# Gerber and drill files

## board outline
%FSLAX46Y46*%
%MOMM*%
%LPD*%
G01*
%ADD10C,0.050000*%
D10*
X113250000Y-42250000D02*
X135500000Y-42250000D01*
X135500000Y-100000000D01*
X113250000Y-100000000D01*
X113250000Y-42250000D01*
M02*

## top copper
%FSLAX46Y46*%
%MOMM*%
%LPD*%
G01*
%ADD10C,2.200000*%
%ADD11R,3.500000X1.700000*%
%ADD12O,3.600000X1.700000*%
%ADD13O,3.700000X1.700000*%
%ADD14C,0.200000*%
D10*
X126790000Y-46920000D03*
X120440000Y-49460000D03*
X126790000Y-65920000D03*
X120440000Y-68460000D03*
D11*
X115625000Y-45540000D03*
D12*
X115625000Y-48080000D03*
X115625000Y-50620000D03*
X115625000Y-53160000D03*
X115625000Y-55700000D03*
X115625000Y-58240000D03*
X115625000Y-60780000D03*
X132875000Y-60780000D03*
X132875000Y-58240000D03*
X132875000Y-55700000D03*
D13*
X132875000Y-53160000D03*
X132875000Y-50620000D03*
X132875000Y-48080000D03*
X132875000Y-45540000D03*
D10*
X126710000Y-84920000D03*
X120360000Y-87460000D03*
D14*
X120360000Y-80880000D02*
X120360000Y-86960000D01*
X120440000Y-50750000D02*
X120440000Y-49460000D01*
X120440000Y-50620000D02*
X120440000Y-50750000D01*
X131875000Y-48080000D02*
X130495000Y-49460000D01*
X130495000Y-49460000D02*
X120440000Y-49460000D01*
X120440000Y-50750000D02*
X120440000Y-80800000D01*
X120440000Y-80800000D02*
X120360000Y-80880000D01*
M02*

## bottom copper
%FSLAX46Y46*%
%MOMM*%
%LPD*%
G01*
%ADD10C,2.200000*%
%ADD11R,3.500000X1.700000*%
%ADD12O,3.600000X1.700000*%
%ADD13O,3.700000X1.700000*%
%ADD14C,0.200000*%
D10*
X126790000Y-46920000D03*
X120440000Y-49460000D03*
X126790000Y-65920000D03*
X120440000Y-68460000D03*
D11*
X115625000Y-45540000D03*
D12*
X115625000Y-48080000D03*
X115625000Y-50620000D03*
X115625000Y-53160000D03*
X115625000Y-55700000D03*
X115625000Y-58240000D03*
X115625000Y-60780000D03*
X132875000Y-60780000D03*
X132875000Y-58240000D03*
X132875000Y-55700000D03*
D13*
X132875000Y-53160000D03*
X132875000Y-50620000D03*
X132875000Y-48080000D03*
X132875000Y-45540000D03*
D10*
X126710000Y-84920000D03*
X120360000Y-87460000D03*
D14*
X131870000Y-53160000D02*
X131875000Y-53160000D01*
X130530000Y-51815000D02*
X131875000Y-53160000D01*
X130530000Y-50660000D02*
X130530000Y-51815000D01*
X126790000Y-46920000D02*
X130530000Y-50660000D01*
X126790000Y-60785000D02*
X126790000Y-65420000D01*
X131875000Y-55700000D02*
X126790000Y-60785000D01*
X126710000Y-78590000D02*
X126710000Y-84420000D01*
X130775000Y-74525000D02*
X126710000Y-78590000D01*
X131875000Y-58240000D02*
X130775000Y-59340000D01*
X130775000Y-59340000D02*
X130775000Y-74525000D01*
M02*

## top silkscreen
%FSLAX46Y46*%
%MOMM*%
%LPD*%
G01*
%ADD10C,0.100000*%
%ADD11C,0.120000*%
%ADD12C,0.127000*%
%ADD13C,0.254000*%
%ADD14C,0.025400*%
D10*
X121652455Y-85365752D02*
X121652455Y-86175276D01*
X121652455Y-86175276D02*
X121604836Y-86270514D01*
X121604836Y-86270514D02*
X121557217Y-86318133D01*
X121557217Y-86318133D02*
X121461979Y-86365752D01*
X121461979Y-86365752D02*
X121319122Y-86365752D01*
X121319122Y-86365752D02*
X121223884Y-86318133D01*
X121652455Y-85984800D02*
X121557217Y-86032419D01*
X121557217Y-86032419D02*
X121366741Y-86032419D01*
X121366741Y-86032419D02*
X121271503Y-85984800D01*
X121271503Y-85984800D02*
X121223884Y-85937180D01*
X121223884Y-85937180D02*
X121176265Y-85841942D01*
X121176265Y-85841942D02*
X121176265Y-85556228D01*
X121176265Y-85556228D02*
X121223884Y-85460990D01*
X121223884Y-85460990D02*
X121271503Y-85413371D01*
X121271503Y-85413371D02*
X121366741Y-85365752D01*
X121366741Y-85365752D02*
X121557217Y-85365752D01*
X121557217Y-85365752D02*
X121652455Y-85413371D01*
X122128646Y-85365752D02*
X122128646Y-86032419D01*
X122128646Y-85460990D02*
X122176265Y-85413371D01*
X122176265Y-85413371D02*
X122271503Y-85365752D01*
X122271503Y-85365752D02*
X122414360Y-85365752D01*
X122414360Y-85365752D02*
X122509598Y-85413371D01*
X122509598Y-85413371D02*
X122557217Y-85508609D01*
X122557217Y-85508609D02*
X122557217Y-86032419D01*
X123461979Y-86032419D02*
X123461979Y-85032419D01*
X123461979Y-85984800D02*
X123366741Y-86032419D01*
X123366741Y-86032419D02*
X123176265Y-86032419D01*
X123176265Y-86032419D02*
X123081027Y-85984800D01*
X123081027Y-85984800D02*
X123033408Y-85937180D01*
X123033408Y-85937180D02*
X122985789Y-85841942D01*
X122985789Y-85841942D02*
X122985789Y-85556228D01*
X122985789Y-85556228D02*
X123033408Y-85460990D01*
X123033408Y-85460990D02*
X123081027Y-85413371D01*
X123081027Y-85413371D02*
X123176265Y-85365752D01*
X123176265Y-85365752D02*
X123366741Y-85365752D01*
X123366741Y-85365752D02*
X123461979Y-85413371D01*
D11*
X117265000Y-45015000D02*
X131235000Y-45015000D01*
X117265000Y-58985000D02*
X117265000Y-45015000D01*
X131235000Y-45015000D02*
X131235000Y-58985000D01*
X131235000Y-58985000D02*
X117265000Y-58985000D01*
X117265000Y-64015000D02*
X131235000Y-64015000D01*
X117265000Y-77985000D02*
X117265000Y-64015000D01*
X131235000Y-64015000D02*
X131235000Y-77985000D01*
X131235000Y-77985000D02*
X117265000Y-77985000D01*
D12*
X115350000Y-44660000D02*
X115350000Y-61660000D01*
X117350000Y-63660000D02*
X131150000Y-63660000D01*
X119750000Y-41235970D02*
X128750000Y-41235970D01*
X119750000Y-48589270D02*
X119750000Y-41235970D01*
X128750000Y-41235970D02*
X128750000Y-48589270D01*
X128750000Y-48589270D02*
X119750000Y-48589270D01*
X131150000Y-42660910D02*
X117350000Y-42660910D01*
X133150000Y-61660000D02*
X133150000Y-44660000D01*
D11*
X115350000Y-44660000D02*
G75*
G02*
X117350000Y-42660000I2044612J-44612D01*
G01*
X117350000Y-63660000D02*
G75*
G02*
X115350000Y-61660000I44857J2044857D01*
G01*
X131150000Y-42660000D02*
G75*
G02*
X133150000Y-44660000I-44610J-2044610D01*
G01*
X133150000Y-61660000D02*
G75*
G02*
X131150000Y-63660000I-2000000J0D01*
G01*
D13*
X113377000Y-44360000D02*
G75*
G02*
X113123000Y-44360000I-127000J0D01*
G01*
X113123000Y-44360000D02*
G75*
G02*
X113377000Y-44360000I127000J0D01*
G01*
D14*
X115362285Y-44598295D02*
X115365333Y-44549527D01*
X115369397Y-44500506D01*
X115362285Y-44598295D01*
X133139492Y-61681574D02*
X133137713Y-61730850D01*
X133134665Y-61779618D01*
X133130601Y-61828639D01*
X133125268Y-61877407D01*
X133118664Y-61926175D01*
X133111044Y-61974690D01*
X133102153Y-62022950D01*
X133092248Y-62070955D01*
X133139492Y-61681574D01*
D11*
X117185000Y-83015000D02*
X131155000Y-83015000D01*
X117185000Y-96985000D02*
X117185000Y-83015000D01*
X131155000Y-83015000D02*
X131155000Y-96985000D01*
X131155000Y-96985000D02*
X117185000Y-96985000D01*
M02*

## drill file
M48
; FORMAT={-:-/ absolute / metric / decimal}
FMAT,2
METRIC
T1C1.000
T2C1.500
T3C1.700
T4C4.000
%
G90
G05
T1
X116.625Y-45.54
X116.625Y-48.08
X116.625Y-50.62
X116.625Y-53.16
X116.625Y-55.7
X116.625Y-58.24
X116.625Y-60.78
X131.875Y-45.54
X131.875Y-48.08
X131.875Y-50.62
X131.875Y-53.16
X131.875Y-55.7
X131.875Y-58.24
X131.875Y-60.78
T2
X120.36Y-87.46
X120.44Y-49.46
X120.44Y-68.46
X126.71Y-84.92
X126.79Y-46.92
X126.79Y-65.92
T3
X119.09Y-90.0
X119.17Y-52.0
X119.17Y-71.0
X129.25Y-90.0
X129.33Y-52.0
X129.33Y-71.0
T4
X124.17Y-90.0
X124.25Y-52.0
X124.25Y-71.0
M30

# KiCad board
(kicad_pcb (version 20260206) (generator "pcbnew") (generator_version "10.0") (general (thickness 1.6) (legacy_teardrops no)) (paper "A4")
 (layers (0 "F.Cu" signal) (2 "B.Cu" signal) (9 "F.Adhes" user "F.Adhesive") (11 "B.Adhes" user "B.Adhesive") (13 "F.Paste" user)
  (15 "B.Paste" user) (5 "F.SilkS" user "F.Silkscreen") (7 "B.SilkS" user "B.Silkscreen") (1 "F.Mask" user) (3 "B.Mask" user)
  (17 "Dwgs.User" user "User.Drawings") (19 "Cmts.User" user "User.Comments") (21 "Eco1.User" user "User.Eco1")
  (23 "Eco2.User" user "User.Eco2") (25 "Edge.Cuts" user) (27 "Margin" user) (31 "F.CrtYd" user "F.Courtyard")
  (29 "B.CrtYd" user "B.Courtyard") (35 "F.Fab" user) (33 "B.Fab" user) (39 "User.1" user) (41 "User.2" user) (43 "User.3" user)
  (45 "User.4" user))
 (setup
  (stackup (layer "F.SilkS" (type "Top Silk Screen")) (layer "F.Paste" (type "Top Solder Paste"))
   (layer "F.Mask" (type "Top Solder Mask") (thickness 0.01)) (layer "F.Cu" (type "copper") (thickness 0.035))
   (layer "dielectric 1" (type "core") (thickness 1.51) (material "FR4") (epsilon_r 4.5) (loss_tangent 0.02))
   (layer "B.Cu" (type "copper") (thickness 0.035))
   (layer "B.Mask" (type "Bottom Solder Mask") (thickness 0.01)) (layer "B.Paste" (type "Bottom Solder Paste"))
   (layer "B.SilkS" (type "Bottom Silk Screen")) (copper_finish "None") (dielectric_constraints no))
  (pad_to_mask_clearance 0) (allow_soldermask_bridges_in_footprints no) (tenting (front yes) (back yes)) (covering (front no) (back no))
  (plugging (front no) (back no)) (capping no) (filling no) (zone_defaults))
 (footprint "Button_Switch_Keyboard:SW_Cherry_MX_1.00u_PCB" (layer "F.Cu") (at 126.79 46.92)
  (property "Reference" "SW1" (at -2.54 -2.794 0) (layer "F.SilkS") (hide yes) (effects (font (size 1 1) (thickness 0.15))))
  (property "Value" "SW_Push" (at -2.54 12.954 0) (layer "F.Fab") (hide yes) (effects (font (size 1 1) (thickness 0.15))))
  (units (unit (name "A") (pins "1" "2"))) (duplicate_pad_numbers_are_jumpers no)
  (fp_line (start -9.525 -1.905) (end 4.445 -1.905) (stroke (width 0.12) (type solid)) (layer "F.SilkS"))
  (fp_line (start -9.525 12.065) (end -9.525 -1.905) (stroke (width 0.12) (type solid)) (layer "F.SilkS"))
  (fp_line (start 4.445 -1.905) (end 4.445 12.065) (stroke (width 0.12) (type solid)) (layer "F.SilkS"))
  (fp_line (start 4.445 12.065) (end -9.525 12.065) (stroke (width 0.12) (type solid)) (layer "F.SilkS"))
  (pad "" np_thru_hole circle (at -7.62 5.08) (size 1.7 1.7) (drill 1.7) (layers "*.Cu" "*.Mask"))
  (pad "" np_thru_hole circle (at -2.54 5.08) (size 4 4) (drill 4) (layers "*.Cu" "*.Mask"))
  (pad "" np_thru_hole circle (at 2.54 5.08) (size 1.7 1.7) (drill 1.7) (layers "*.Cu" "*.Mask"))
  (pad "1" thru_hole circle (at 0 0) (size 2.2 2.2) (drill 1.5) (layers "*.Cu" "*.Mask") (remove_unused_layers no)
   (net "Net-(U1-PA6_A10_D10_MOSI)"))
  (pad "2" thru_hole circle (at -6.35 2.54) (size 2.2 2.2) (drill 1.5) (layers "*.Cu" "*.Mask") (remove_unused_layers no) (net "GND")))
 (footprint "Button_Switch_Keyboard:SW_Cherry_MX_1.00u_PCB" (layer "F.Cu") (at 126.79 65.92)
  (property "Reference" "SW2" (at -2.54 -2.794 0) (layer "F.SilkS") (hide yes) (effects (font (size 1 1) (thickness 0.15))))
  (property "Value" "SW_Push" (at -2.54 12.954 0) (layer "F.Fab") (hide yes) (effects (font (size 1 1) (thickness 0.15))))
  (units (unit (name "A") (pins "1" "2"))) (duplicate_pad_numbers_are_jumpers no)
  (fp_line (start -9.525 -1.905) (end 4.445 -1.905) (stroke (width 0.12) (type solid)) (layer "F.SilkS"))
  (fp_line (start -9.525 12.065) (end -9.525 -1.905) (stroke (width 0.12) (type solid)) (layer "F.SilkS"))
  (fp_line (start 4.445 -1.905) (end 4.445 12.065) (stroke (width 0.12) (type solid)) (layer "F.SilkS"))
  (fp_line (start 4.445 12.065) (end -9.525 12.065) (stroke (width 0.12) (type solid)) (layer "F.SilkS"))
  (pad "" np_thru_hole circle (at -7.62 5.08) (size 1.7 1.7) (drill 1.7) (layers "*.Cu" "*.Mask"))
  (pad "" np_thru_hole circle (at -2.54 5.08) (size 4 4) (drill 4) (layers "*.Cu" "*.Mask"))
  (pad "" np_thru_hole circle (at 2.54 5.08) (size 1.7 1.7) (drill 1.7) (layers "*.Cu" "*.Mask"))
  (pad "1" thru_hole circle (at 0 0) (size 2.2 2.2) (drill 1.5) (layers "*.Cu" "*.Mask") (remove_unused_layers no)
   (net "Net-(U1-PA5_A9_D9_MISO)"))
  (pad "2" thru_hole circle (at -6.35 2.54) (size 2.2 2.2) (drill 1.5) (layers "*.Cu" "*.Mask") (remove_unused_layers no) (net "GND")))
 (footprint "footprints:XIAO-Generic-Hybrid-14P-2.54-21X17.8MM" (layer "F.Cu") (at 124.25 53.16)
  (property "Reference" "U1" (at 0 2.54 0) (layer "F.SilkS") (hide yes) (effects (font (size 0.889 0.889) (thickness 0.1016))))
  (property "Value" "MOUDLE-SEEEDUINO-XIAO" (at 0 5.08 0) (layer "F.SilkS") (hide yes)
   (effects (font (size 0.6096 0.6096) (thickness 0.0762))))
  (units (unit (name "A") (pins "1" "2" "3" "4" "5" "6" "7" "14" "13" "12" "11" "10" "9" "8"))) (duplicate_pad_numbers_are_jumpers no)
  (fp_line (start -8.9 -8.5) (end -8.9 8.5) (stroke (width 0.127) (type solid)) (layer "F.SilkS"))
  (fp_line (start -6.9 10.5) (end 6.9 10.5) (stroke (width 0.127) (type solid)) (layer "F.SilkS"))
  (fp_line (start -4.5 -11.92403) (end 4.5 -11.92403) (stroke (width 0.127) (type solid)) (layer "F.SilkS"))
  (fp_line (start -4.5 -4.57073) (end -4.5 -11.92403) (stroke (width 0.127) (type solid)) (layer "F.SilkS"))
  (fp_line (start 4.5 -11.92403) (end 4.5 -4.57073) (stroke (width 0.127) (type solid)) (layer "F.SilkS"))
  (fp_line (start 4.5 -4.57073) (end -4.5 -4.57073) (stroke (width 0.127) (type solid)) (layer "F.SilkS"))
  (fp_line (start 6.9 -10.49909) (end -6.9 -10.49909) (stroke (width 0.127) (type solid)) (layer "F.SilkS"))
  (fp_line (start 8.9 8.5) (end 8.9 -8.5) (stroke (width 0.127) (type solid)) (layer "F.SilkS"))
  (fp_arc (start -8.9 -8.5) (mid -8.301491 -9.901491) (end -6.9 -10.5) (stroke (width 0.12) (type solid)) (layer "F.SilkS"))
  (fp_arc (start -6.9 10.5) (mid -8.301423 9.901423) (end -8.9 8.5) (stroke (width 0.12) (type solid)) (layer "F.SilkS"))
  (fp_arc (start 6.9 -10.5) (mid 8.301491 -9.901491) (end 8.9 -8.5) (stroke (width 0.12) (type solid)) (layer "F.SilkS"))
  (fp_arc (start 8.9 8.5) (mid 8.314214 9.914214) (end 6.9 10.5) (stroke (width 0.12) (type solid)) (layer "F.SilkS"))
  (fp_circle (center -11 -8.8) (end -11 -9.054) (stroke (width 0) (type solid)) (fill yes) (layer "F.SilkS"))
  (fp_poly
   (pts (xy -8.887715 -8.561705) (xy -8.884667 -8.610473) (xy -8.880603 -8.659494)) (stroke (width 0.0254) (type solid)) (fill no)
   (layer "F.SilkS"))
  (fp_poly
   (pts (xy 8.889492 8.521574) (xy 8.887713 8.57085) (xy 8.884665 8.619618) (xy 8.880601 8.668639) (xy 8.875268 8.717407)
    (xy 8.868664 8.766175) (xy 8.861044 8.81469) (xy 8.852153 8.86295) (xy 8.842248 8.910955))
   (stroke (width 0.0254) (type solid)) (fill no) (layer "F.SilkS"))
  (pad "1" thru_hole rect (at -7.625 -7.62) (size 3.5 1.7) (drill 1 (offset -1 0)) (layers "*.Cu" "*.Mask") (remove_unused_layers no)
   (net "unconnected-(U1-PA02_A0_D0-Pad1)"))
  (pad "2" thru_hole oval (at -7.625 -5.08) (size 3.6 1.7) (drill 1 (offset -1 0)) (layers "*.Cu" "*.Mask") (remove_unused_layers no)
   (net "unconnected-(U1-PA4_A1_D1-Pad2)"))
  (pad "3" thru_hole oval (at -7.625 -2.54) (size 3.6 1.7) (drill 1 (offset -1 0)) (layers "*.Cu" "*.Mask") (remove_unused_layers no)
   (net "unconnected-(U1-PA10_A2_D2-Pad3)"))
  (pad "4" thru_hole oval (at -7.625 0) (size 3.6 1.7) (drill 1 (offset -1 0)) (layers "*.Cu" "*.Mask") (remove_unused_layers no)
   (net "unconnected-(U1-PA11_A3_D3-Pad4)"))
  (pad "5" thru_hole oval (at -7.625 2.54) (size 3.6 1.7) (drill 1 (offset -1 0)) (layers "*.Cu" "*.Mask") (remove_unused_layers no)
   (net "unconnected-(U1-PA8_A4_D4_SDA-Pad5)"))
  (pad "6" thru_hole oval (at -7.625 5.08 180) (size 3.6 1.7) (drill 1 (offset 1 0)) (layers "*.Cu" "*.Mask") (remove_unused_layers no)
   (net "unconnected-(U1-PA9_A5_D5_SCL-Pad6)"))
  (pad "7" thru_hole oval (at -7.625 7.62) (size 3.6 1.7) (drill 1 (offset -1 0)) (layers "*.Cu" "*.Mask") (remove_unused_layers no)
   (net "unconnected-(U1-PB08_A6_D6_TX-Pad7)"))
  (pad "8" thru_hole oval (at 7.625 7.62) (size 3.6 1.7) (drill 1 (offset 1 0)) (layers "*.Cu" "*.Mask") (remove_unused_layers no)
   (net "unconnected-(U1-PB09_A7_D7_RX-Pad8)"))
  (pad "9" thru_hole oval (at 7.625 5.08) (size 3.6 1.7) (drill 1 (offset 1 0)) (layers "*.Cu" "*.Mask") (remove_unused_layers no)
   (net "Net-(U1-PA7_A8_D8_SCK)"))
  (pad "10" thru_hole oval (at 7.625 2.54) (size 3.6 1.7) (drill 1 (offset 1 0)) (layers "*.Cu" "*.Mask") (remove_unused_layers no)
   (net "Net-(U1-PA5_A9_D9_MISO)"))
  (pad "11" thru_hole oval (at 7.625 0) (size 3.7 1.7) (drill 1 (offset 1 0)) (layers "*.Cu" "*.Mask") (remove_unused_layers no)
   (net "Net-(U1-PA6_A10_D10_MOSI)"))
  (pad "12" thru_hole oval (at 7.625 -2.54) (size 3.7 1.7) (drill 1 (offset 1 0)) (layers "*.Cu" "*.Mask") (remove_unused_layers no)
   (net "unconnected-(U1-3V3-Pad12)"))
  (pad "13" thru_hole oval (at 7.625 -5.08) (size 3.7 1.7) (drill 1 (offset 1 0)) (layers "*.Cu" "*.Mask") (remove_unused_layers no)
   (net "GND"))
  (pad "14" thru_hole oval (at 7.625 -7.62) (size 3.7 1.7) (drill 1 (offset 1 0)) (layers "*.Cu" "*.Mask") (remove_unused_layers no)
   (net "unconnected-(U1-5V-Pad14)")))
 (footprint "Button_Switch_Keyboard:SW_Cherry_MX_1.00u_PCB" (layer "F.Cu") (at 126.71 84.92)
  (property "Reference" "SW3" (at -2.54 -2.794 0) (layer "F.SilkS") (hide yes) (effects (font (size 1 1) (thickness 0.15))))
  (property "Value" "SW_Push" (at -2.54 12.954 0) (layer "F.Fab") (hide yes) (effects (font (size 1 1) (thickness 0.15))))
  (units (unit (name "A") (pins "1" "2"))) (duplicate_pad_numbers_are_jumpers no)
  (fp_line (start -9.525 -1.905) (end 4.445 -1.905) (stroke (width 0.12) (type solid)) (layer "F.SilkS"))
  (fp_line (start -9.525 12.065) (end -9.525 -1.905) (stroke (width 0.12) (type solid)) (layer "F.SilkS"))
  (fp_line (start 4.445 -1.905) (end 4.445 12.065) (stroke (width 0.12) (type solid)) (layer "F.SilkS"))
  (fp_line (start 4.445 12.065) (end -9.525 12.065) (stroke (width 0.12) (type solid)) (layer "F.SilkS"))
  (pad "" np_thru_hole circle (at -7.62 5.08) (size 1.7 1.7) (drill 1.7) (layers "*.Cu" "*.Mask"))
  (pad "" np_thru_hole circle (at -2.54 5.08) (size 4 4) (drill 4) (layers "*.Cu" "*.Mask"))
  (pad "" np_thru_hole circle (at 2.54 5.08) (size 1.7 1.7) (drill 1.7) (layers "*.Cu" "*.Mask"))
  (pad "1" thru_hole circle (at 0 0) (size 2.2 2.2) (drill 1.5) (layers "*.Cu" "*.Mask") (remove_unused_layers no)
   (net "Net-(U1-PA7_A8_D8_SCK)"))
  (pad "2" thru_hole circle (at -6.35 2.54) (size 2.2 2.2) (drill 1.5) (layers "*.Cu" "*.Mask") (remove_unused_layers no) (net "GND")))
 (gr_rect (start 113.25 42.25) (end 135.5 100) (stroke (width 0.05) (type default)) (fill no) (layer "Edge.Cuts"))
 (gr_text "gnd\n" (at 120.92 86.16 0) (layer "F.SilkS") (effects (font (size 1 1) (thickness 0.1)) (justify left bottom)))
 (segment (start 131.87 53.16) (end 131.875 53.16) (width 0.2) (layer "B.Cu") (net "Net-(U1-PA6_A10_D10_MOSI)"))
 (segment (start 130.53 51.815) (end 131.875 53.16) (width 0.2) (layer "B.Cu") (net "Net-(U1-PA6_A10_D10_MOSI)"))
 (segment (start 130.53 50.66) (end 130.53 51.815) (width 0.2) (layer "B.Cu") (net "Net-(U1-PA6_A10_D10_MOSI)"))
 (segment (start 126.79 46.92) (end 130.53 50.66) (width 0.2) (layer "B.Cu") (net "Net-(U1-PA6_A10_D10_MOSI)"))
 (segment (start 120.36 80.88) (end 120.36 86.96) (width 0.2) (layer "F.Cu") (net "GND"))
 (segment (start 120.44 50.75) (end 120.44 49.46) (width 0.2) (layer "F.Cu") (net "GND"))
 (segment (start 120.44 50.62) (end 120.44 50.75) (width 0.2) (layer "F.Cu") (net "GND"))
 (segment (start 131.875 48.08) (end 130.495 49.46) (width 0.2) (layer "F.Cu") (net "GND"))
 (segment (start 130.495 49.46) (end 120.44 49.46) (width 0.2) (layer "F.Cu") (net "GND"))
 (segment (start 120.44 50.75) (end 120.44 80.8) (width 0.2) (layer "F.Cu") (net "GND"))
 (segment (start 120.44 80.8) (end 120.36 80.88) (width 0.2) (layer "F.Cu") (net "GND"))
 (segment (start 126.79 60.785) (end 126.79 65.42) (width 0.2) (layer "B.Cu") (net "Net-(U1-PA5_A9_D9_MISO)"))
 (segment (start 131.875 55.7) (end 126.79 60.785) (width 0.2) (layer "B.Cu") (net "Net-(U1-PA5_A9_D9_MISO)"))
 (segment (start 126.71 78.59) (end 126.71 84.42) (width 0.2) (layer "B.Cu") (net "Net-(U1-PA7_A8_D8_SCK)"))
 (segment (start 130.775 74.525) (end 126.71 78.59) (width 0.2) (layer "B.Cu") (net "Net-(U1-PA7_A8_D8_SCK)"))
 (segment (start 131.875 58.24) (end 130.775 59.34) (width 0.2) (layer "B.Cu") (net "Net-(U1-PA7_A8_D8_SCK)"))
 (segment (start 130.775 59.34) (end 130.775 74.525) (width 0.2) (layer "B.Cu") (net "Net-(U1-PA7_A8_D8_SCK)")))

